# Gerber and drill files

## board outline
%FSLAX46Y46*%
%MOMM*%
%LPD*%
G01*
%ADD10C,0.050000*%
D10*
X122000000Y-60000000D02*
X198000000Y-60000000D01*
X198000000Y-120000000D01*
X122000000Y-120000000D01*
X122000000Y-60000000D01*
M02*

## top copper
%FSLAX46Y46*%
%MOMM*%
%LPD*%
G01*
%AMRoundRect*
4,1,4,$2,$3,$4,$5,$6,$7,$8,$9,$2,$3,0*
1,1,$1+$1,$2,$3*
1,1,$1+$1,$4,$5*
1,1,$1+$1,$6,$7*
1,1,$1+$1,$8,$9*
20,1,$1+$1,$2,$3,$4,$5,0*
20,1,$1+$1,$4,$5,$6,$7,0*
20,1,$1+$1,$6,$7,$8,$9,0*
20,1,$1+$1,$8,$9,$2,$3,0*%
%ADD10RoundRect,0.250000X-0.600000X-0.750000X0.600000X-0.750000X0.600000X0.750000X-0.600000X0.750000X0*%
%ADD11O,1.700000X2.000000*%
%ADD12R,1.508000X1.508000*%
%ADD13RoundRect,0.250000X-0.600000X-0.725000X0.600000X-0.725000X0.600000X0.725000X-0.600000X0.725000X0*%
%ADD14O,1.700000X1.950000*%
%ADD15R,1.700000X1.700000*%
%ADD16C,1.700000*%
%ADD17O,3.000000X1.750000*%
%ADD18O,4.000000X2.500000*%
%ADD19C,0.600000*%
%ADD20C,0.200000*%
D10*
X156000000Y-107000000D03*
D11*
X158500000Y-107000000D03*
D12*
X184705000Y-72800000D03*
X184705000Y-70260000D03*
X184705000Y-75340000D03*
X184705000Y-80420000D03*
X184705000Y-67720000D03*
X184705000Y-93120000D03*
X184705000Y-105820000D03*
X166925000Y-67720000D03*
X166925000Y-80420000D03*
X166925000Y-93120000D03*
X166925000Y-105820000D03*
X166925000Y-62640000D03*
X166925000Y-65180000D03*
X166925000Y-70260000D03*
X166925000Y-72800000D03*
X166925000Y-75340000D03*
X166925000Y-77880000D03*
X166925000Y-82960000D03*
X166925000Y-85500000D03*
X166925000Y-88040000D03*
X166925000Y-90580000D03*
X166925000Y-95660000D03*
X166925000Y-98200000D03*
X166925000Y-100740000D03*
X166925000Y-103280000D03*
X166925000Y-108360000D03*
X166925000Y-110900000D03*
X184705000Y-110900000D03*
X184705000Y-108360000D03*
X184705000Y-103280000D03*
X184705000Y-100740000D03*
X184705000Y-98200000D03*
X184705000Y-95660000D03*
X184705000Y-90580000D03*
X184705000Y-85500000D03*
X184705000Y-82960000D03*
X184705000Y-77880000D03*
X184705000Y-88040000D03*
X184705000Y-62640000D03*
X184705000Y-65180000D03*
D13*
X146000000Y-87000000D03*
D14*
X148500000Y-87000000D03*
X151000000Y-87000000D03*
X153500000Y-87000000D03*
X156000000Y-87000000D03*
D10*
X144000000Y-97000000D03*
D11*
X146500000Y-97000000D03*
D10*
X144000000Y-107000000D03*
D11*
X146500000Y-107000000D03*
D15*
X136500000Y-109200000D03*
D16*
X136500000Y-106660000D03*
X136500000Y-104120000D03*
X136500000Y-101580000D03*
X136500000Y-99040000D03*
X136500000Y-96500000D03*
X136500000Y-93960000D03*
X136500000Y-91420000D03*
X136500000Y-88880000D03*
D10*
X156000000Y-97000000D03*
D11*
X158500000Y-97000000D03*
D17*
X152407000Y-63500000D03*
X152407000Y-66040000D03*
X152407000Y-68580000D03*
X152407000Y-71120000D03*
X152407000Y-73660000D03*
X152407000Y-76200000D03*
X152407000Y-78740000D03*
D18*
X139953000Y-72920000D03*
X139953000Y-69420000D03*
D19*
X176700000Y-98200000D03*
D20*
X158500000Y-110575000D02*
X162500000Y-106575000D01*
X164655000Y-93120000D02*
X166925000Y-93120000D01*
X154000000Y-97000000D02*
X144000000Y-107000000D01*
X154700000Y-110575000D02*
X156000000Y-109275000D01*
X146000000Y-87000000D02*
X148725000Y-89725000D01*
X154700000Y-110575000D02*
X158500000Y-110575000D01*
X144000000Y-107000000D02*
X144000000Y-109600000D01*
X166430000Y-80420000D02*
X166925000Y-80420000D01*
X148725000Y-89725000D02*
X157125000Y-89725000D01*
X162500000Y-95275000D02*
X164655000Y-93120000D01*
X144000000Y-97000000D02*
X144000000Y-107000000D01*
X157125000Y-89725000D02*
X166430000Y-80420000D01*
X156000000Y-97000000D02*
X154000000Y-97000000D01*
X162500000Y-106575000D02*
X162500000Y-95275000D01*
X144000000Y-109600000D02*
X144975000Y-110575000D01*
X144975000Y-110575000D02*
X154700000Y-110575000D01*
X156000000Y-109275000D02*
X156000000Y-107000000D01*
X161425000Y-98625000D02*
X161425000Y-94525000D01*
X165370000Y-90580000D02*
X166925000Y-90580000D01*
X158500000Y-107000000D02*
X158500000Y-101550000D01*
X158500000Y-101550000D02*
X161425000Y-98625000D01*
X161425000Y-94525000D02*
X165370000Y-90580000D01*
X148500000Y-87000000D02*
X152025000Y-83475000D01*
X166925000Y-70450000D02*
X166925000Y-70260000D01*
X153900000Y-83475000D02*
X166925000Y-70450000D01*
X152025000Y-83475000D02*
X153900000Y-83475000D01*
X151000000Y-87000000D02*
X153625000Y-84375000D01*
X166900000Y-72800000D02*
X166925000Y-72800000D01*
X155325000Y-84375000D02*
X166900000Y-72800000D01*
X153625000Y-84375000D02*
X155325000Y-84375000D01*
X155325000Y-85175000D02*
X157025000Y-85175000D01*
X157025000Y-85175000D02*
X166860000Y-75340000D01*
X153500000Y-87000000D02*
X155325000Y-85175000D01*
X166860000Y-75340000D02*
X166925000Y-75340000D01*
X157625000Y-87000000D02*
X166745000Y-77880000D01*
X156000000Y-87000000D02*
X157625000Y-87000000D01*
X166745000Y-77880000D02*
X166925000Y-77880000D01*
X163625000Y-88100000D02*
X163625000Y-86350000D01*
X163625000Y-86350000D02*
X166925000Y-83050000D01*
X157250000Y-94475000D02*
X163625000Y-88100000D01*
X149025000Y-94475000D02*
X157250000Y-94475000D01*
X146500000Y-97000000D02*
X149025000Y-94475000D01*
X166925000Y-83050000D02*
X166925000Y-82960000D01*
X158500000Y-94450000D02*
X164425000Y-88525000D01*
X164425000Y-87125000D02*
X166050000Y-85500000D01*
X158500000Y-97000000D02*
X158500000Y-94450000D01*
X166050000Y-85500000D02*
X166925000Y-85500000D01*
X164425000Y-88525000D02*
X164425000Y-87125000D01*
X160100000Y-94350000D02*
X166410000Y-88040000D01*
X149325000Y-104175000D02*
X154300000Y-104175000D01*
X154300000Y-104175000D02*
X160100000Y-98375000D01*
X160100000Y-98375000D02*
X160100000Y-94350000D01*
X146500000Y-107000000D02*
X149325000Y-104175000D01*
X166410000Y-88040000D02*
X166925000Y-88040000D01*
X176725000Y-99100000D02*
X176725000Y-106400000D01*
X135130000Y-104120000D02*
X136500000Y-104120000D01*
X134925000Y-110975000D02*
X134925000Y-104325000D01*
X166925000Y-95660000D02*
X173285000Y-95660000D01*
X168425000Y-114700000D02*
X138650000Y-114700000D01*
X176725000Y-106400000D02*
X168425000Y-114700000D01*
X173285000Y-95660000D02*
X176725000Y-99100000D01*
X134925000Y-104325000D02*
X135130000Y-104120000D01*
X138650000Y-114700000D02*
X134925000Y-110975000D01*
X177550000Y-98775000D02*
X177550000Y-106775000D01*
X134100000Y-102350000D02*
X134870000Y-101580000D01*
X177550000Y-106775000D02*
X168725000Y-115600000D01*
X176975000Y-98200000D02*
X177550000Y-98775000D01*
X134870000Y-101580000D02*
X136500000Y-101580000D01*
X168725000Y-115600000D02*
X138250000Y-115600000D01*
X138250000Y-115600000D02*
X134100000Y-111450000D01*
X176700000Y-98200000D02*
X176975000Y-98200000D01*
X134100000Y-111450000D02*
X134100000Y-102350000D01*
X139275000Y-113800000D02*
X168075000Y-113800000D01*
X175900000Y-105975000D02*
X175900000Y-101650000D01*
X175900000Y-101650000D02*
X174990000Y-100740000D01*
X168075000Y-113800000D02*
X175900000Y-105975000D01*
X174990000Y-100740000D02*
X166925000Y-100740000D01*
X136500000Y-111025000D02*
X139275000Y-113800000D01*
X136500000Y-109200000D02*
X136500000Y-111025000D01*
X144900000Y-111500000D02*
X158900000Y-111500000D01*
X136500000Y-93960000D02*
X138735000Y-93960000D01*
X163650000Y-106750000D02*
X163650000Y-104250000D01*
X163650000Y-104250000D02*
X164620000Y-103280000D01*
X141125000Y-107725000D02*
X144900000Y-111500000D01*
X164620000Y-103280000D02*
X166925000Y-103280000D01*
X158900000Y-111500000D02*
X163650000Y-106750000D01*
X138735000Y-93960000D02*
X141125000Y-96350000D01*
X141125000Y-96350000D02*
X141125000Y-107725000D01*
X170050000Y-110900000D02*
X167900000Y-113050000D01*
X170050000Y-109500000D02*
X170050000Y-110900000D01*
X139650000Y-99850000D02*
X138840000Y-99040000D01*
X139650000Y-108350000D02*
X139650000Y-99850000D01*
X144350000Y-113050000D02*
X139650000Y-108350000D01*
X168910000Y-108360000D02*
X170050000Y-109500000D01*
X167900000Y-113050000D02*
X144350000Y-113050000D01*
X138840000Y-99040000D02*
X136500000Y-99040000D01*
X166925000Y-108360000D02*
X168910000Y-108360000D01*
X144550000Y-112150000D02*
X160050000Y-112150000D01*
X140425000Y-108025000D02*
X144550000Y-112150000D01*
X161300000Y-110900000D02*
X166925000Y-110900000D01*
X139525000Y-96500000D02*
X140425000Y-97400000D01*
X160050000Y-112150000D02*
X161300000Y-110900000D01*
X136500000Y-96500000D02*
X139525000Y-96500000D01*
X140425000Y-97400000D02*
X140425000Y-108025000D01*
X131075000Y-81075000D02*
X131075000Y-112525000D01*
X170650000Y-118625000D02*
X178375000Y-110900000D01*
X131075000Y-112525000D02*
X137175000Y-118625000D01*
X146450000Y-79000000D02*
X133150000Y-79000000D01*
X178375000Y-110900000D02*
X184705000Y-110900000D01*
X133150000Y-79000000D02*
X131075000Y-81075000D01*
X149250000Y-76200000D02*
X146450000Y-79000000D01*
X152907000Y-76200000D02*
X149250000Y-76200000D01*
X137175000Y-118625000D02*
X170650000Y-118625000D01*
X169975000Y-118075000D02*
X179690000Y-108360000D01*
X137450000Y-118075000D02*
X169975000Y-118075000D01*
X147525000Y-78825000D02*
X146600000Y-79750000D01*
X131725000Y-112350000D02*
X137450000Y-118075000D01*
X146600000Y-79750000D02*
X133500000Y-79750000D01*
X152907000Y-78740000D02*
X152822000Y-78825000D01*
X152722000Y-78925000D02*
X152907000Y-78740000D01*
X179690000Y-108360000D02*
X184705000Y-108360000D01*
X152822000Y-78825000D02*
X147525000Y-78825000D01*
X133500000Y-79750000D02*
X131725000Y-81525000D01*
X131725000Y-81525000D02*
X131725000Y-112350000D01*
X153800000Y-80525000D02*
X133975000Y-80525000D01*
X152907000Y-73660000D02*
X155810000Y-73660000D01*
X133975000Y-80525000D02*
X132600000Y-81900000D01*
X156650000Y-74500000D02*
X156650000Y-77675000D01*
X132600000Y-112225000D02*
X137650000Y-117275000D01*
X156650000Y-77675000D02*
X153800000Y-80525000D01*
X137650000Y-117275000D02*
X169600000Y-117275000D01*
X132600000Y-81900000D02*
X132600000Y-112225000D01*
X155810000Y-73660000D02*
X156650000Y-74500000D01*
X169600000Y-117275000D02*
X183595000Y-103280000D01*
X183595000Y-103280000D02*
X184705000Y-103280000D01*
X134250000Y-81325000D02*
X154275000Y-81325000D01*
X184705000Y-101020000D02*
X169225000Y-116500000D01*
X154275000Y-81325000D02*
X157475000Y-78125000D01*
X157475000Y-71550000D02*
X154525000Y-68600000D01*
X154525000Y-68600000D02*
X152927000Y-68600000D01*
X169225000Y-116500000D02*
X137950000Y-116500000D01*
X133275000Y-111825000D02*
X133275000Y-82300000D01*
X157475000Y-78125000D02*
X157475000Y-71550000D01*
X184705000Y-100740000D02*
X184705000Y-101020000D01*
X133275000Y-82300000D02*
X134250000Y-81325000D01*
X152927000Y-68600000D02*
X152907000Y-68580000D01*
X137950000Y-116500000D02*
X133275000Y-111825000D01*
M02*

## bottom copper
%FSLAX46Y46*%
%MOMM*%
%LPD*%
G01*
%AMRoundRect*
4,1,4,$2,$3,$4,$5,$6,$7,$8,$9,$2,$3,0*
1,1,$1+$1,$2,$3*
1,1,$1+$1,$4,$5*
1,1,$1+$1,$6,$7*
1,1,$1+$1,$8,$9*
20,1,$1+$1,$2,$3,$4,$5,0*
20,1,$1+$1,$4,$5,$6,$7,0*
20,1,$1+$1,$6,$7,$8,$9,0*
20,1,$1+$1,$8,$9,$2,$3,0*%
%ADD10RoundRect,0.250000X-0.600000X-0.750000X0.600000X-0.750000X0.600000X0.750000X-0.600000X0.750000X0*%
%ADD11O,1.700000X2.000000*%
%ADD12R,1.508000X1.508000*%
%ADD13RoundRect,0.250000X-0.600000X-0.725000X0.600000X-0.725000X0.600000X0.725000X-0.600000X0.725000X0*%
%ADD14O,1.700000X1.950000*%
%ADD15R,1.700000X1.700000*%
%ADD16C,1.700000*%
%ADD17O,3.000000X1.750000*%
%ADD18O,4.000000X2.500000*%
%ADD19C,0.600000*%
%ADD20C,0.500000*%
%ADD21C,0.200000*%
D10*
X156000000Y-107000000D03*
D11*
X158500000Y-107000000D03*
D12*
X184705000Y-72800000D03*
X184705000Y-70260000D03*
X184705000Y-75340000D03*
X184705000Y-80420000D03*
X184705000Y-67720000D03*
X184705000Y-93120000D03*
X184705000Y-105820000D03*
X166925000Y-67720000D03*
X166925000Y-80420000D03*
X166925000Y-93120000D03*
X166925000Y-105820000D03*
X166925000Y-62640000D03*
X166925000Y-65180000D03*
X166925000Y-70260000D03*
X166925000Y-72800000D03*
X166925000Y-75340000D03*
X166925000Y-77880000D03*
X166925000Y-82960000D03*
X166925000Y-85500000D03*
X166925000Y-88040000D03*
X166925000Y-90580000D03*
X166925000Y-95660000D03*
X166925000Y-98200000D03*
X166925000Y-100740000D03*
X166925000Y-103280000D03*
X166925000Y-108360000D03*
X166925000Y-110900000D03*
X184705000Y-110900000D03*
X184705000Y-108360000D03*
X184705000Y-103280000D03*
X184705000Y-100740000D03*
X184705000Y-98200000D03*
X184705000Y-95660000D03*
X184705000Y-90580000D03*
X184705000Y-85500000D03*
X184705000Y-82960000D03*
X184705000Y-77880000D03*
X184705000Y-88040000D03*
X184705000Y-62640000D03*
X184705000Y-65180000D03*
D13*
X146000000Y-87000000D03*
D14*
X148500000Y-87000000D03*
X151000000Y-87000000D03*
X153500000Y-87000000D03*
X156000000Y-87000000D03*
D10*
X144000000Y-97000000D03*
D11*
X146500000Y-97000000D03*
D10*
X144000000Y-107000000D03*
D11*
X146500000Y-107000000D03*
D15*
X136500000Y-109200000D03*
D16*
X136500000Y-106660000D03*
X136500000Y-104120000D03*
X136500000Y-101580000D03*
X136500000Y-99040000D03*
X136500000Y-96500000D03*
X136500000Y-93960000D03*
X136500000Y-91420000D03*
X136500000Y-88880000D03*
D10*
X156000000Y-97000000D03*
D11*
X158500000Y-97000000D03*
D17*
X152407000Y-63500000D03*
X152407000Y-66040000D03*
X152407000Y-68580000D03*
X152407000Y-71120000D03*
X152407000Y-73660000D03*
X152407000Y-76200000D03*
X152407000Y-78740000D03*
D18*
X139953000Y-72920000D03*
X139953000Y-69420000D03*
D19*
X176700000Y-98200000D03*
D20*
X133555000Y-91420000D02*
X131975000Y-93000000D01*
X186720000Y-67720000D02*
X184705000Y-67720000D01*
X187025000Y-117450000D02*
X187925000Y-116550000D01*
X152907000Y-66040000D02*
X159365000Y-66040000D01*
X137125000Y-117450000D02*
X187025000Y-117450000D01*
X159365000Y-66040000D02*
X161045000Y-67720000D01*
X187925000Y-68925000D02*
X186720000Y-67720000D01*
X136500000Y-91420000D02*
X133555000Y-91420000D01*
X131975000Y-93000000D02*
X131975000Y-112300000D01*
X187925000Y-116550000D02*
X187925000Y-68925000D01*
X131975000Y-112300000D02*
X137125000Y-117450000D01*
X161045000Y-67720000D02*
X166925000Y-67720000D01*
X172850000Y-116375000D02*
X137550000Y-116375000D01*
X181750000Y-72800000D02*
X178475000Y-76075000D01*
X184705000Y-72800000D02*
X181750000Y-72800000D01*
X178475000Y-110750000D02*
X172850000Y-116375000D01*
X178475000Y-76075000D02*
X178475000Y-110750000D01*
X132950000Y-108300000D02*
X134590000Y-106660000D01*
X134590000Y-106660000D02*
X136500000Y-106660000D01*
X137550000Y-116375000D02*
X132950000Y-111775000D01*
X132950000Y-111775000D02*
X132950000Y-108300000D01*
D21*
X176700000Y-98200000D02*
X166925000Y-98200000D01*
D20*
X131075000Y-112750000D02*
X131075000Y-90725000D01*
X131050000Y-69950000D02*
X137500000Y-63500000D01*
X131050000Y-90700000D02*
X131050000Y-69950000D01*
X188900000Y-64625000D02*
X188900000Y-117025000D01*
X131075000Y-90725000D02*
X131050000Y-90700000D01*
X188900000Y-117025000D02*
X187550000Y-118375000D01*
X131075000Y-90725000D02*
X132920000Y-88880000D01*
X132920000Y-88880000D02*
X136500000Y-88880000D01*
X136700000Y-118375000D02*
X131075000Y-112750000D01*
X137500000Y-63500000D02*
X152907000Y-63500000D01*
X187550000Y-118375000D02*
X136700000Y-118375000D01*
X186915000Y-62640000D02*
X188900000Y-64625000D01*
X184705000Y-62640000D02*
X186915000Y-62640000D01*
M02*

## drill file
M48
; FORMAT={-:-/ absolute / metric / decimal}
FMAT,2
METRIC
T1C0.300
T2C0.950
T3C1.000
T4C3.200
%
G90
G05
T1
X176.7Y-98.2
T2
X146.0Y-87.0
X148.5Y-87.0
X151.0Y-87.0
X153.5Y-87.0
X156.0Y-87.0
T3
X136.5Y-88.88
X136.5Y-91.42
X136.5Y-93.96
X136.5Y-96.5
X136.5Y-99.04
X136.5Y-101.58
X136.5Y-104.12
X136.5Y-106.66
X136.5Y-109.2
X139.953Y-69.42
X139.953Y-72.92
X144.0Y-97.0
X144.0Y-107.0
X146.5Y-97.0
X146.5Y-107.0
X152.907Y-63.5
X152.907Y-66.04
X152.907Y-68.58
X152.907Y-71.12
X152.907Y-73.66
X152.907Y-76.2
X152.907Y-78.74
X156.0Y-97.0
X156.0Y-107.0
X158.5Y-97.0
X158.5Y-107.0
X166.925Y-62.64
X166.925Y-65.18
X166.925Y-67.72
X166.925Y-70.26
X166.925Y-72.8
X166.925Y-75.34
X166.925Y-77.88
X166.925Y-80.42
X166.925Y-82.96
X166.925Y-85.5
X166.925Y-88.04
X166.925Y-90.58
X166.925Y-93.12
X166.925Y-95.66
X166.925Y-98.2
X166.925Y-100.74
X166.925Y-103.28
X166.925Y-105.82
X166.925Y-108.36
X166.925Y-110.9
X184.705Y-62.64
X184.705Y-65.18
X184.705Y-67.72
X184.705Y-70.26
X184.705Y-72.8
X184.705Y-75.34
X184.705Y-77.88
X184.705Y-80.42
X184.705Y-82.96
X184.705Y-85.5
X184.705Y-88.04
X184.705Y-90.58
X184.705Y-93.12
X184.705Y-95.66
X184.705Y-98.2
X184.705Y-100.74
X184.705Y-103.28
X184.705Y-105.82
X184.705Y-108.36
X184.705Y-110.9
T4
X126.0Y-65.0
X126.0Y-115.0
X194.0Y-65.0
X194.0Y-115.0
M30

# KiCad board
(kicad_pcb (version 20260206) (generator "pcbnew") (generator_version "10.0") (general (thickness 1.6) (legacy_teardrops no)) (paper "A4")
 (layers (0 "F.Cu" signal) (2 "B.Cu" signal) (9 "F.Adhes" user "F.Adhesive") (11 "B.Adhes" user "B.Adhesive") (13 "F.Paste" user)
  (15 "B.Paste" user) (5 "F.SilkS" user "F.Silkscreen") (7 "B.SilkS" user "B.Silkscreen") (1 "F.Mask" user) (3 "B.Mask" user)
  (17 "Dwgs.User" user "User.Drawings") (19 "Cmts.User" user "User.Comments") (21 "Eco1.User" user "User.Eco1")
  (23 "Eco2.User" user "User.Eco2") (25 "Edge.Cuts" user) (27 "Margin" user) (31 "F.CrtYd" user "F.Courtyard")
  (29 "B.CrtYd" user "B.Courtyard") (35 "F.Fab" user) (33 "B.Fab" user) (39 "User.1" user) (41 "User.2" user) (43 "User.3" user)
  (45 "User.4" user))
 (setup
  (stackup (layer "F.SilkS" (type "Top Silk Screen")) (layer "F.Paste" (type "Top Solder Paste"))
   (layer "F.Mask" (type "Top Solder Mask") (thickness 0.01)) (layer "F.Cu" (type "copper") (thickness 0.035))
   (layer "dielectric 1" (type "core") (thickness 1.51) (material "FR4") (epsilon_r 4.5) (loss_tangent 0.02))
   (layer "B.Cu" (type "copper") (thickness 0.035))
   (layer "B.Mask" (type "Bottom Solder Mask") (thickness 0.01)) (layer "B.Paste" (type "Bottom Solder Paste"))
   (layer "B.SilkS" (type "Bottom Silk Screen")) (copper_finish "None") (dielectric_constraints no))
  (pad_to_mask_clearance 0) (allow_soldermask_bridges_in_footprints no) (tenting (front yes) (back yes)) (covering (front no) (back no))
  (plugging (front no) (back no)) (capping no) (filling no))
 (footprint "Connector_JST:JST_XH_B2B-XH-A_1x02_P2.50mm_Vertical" (layer "F.Cu") (at 156 107)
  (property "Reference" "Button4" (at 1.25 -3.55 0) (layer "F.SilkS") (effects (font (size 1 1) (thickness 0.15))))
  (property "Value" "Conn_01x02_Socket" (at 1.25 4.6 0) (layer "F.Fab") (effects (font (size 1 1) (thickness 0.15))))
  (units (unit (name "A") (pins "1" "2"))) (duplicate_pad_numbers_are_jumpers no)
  (pad "1" thru_hole roundrect (at 0 0) (size 1.7 2) (drill 1) (layers "*.Cu" "*.Mask") (remove_unused_layers no)
   (roundrect_rratio 0.147059) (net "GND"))
  (pad "2" thru_hole oval (at 2.5 0) (size 1.7 2) (drill 1) (layers "*.Cu" "*.Mask") (remove_unused_layers no) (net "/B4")))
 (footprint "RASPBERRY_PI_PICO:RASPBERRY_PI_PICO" (layer "F.Cu") (at 175.815 85.5)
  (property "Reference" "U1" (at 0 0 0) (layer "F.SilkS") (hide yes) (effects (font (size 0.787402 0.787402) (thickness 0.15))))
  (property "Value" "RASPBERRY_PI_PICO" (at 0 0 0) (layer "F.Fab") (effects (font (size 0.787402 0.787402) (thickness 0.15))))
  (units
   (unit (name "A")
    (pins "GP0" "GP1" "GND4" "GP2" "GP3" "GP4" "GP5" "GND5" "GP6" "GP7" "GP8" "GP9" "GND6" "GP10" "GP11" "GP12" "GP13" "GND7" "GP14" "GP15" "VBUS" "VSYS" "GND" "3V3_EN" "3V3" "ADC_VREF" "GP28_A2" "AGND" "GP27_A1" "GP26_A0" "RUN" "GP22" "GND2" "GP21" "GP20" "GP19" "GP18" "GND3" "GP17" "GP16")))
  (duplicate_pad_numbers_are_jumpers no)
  (pad "3V3" thru_hole rect (at 8.89 -12.7) (size 1.508 1.508) (drill 1) (layers "*.Cu" "*.Mask") (remove_unused_layers no) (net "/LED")
   (solder_mask_margin 0.102))
  (pad "3V3_EN" thru_hole rect (at 8.89 -15.24) (size 1.508 1.508) (drill 1) (layers "*.Cu" "*.Mask") (remove_unused_layers no)
   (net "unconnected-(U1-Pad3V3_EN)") (solder_mask_margin 0.102))
  (pad "ADC_VREF" thru_hole rect (at 8.89 -10.16) (size 1.508 1.508) (drill 1) (layers "*.Cu" "*.Mask") (remove_unused_layers no)
   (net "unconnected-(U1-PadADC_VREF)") (solder_mask_margin 0.102))
  (pad "AGND" thru_hole rect (at 8.89 -5.08) (size 1.508 1.508) (drill 1) (layers "*.Cu" "*.Mask") (remove_unused_layers no)
   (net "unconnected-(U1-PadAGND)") (solder_mask_margin 0.102))
  (pad "GND" thru_hole rect (at 8.89 -17.78) (size 1.508 1.508) (drill 1) (layers "*.Cu" "*.Mask") (remove_unused_layers no) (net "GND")
   (solder_mask_margin 0.102))
  (pad "GND2" thru_hole rect (at 8.89 7.62) (size 1.508 1.508) (drill 1) (layers "*.Cu" "*.Mask") (remove_unused_layers no)
   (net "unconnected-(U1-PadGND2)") (solder_mask_margin 0.102))
  (pad "GND3" thru_hole rect (at 8.89 20.32) (size 1.508 1.508) (drill 1) (layers "*.Cu" "*.Mask") (remove_unused_layers no)
   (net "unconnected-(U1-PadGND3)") (solder_mask_margin 0.102))
  (pad "GND4" thru_hole rect (at -8.89 -17.78) (size 1.508 1.508) (drill 1) (layers "*.Cu" "*.Mask") (remove_unused_layers no) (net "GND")
   (solder_mask_margin 0.102))
  (pad "GND5" thru_hole rect (at -8.89 -5.08) (size 1.508 1.508) (drill 1) (layers "*.Cu" "*.Mask") (remove_unused_layers no) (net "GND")
   (solder_mask_margin 0.102))
  (pad "GND6" thru_hole rect (at -8.89 7.62) (size 1.508 1.508) (drill 1) (layers "*.Cu" "*.Mask") (remove_unused_layers no) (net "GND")
   (solder_mask_margin 0.102))
  (pad "GND7" thru_hole rect (at -8.89 20.32) (size 1.508 1.508) (drill 1) (layers "*.Cu" "*.Mask") (remove_unused_layers no)
   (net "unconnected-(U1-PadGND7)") (solder_mask_margin 0.102))
  (pad "GP0" thru_hole rect (at -8.89 -22.86) (size 1.508 1.508) (drill 1) (layers "*.Cu" "*.Mask") (remove_unused_layers no)
   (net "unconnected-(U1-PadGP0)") (solder_mask_margin 0.102))
  (pad "GP1" thru_hole rect (at -8.89 -20.32) (size 1.508 1.508) (drill 1) (layers "*.Cu" "*.Mask") (remove_unused_layers no)
   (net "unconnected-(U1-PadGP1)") (solder_mask_margin 0.102))
  (pad "GP2" thru_hole rect (at -8.89 -15.24) (size 1.508 1.508) (drill 1) (layers "*.Cu" "*.Mask") (remove_unused_layers no) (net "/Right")
   (solder_mask_margin 0.102))
  (pad "GP3" thru_hole rect (at -8.89 -12.7) (size 1.508 1.508) (drill 1) (layers "*.Cu" "*.Mask") (remove_unused_layers no) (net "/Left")
   (solder_mask_margin 0.102))
  (pad "GP4" thru_hole rect (at -8.89 -10.16) (size 1.508 1.508) (drill 1) (layers "*.Cu" "*.Mask") (remove_unused_layers no) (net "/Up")
   (solder_mask_margin 0.102))
  (pad "GP5" thru_hole rect (at -8.89 -7.62) (size 1.508 1.508) (drill 1) (layers "*.Cu" "*.Mask") (remove_unused_layers no) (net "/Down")
   (solder_mask_margin 0.102))
  (pad "GP6" thru_hole rect (at -8.89 -2.54) (size 1.508 1.508) (drill 1) (layers "*.Cu" "*.Mask") (remove_unused_layers no) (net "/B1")
   (solder_mask_margin 0.102))
  (pad "GP7" thru_hole rect (at -8.89 0) (size 1.508 1.508) (drill 1) (layers "*.Cu" "*.Mask") (remove_unused_layers no) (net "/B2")
   (solder_mask_margin 0.102))
  (pad "GP8" thru_hole rect (at -8.89 2.54) (size 1.508 1.508) (drill 1) (layers "*.Cu" "*.Mask") (remove_unused_layers no) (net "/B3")
   (solder_mask_margin 0.102))
  (pad "GP9" thru_hole rect (at -8.89 5.08) (size 1.508 1.508) (drill 1) (layers "*.Cu" "*.Mask") (remove_unused_layers no) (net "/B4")
   (solder_mask_margin 0.102))
  (pad "GP10" thru_hole rect (at -8.89 10.16) (size 1.508 1.508) (drill 1) (layers "*.Cu" "*.Mask") (remove_unused_layers no) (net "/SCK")
   (solder_mask_margin 0.102))
  (pad "GP11" thru_hole rect (at -8.89 12.7) (size 1.508 1.508) (drill 1) (layers "*.Cu" "*.Mask") (remove_unused_layers no) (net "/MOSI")
   (solder_mask_margin 0.102))
  (pad "GP12" thru_hole rect (at -8.89 15.24) (size 1.508 1.508) (drill 1) (layers "*.Cu" "*.Mask") (remove_unused_layers no) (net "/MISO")
   (solder_mask_margin 0.102))
  (pad "GP13" thru_hole rect (at -8.89 17.78) (size 1.508 1.508) (drill 1) (layers "*.Cu" "*.Mask") (remove_unused_layers no) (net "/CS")
   (solder_mask_margin 0.102))
  (pad "GP14" thru_hole rect (at -8.89 22.86) (size 1.508 1.508) (drill 1) (layers "*.Cu" "*.Mask") (remove_unused_layers no)
   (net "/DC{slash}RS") (solder_mask_margin 0.102))
  (pad "GP15" thru_hole rect (at -8.89 25.4) (size 1.508 1.508) (drill 1) (layers "*.Cu" "*.Mask") (remove_unused_layers no) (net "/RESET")
   (solder_mask_margin 0.102))
  (pad "GP16" thru_hole rect (at 8.89 25.4) (size 1.508 1.508) (drill 1) (layers "*.Cu" "*.Mask") (remove_unused_layers no) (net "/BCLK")
   (solder_mask_margin 0.102))
  (pad "GP17" thru_hole rect (at 8.89 22.86) (size 1.508 1.508) (drill 1) (layers "*.Cu" "*.Mask") (remove_unused_layers no) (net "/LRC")
   (solder_mask_margin 0.102))
  (pad "GP18" thru_hole rect (at 8.89 17.78) (size 1.508 1.508) (drill 1) (layers "*.Cu" "*.Mask") (remove_unused_layers no) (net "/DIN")
   (solder_mask_margin 0.102))
  (pad "GP19" thru_hole rect (at 8.89 15.24) (size 1.508 1.508) (drill 1) (layers "*.Cu" "*.Mask") (remove_unused_layers no)
   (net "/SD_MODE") (solder_mask_margin 0.102))
  (pad "GP20" thru_hole rect (at 8.89 12.7) (size 1.508 1.508) (drill 1) (layers "*.Cu" "*.Mask") (remove_unused_layers no)
   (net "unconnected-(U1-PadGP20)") (solder_mask_margin 0.102))
  (pad "GP21" thru_hole rect (at 8.89 10.16) (size 1.508 1.508) (drill 1) (layers "*.Cu" "*.Mask") (remove_unused_layers no)
   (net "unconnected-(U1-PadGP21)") (solder_mask_margin 0.102))
  (pad "GP22" thru_hole rect (at 8.89 5.08) (size 1.508 1.508) (drill 1) (layers "*.Cu" "*.Mask") (remove_unused_layers no)
   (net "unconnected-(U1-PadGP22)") (solder_mask_margin 0.102))
  (pad "GP26_A0" thru_hole rect (at 8.89 0) (size 1.508 1.508) (drill 1) (layers "*.Cu" "*.Mask") (remove_unused_layers no)
   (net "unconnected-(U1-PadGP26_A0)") (solder_mask_margin 0.102))
  (pad "GP27_A1" thru_hole rect (at 8.89 -2.54) (size 1.508 1.508) (drill 1) (layers "*.Cu" "*.Mask") (remove_unused_layers no)
   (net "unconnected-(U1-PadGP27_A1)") (solder_mask_margin 0.102))
  (pad "GP28_A2" thru_hole rect (at 8.89 -7.62) (size 1.508 1.508) (drill 1) (layers "*.Cu" "*.Mask") (remove_unused_layers no)
   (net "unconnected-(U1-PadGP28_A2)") (solder_mask_margin 0.102))
  (pad "RUN" thru_hole rect (at 8.89 2.54) (size 1.508 1.508) (drill 1) (layers "*.Cu" "*.Mask") (remove_unused_layers no)
   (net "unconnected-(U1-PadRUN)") (solder_mask_margin 0.102))
  (pad "VBUS" thru_hole rect (at 8.89 -22.86) (size 1.508 1.508) (drill 1) (layers "*.Cu" "*.Mask") (remove_unused_layers no) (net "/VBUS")
   (solder_mask_margin 0.102))
  (pad "VSYS" thru_hole rect (at 8.89 -20.32) (size 1.508 1.508) (drill 1) (layers "*.Cu" "*.Mask") (remove_unused_layers no)
   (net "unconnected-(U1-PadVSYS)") (solder_mask_margin 0.102)))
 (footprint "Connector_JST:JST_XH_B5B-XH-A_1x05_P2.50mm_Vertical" (layer "F.Cu") (at 146 87)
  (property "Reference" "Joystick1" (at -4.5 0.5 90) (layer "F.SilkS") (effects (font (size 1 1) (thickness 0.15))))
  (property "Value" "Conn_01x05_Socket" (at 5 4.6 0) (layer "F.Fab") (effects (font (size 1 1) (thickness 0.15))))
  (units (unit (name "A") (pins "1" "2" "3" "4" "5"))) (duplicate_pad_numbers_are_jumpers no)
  (pad "1" thru_hole roundrect (at 0 0) (size 1.7 1.95) (drill 0.95) (layers "*.Cu" "*.Mask") (remove_unused_layers no)
   (roundrect_rratio 0.147059) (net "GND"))
  (pad "2" thru_hole oval (at 2.5 0) (size 1.7 1.95) (drill 0.95) (layers "*.Cu" "*.Mask") (remove_unused_layers no) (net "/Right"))
  (pad "3" thru_hole oval (at 5 0) (size 1.7 1.95) (drill 0.95) (layers "*.Cu" "*.Mask") (remove_unused_layers no) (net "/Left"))
  (pad "4" thru_hole oval (at 7.5 0) (size 1.7 1.95) (drill 0.95) (layers "*.Cu" "*.Mask") (remove_unused_layers no) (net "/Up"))
  (pad "5" thru_hole oval (at 10 0) (size 1.7 1.95) (drill 0.95) (layers "*.Cu" "*.Mask") (remove_unused_layers no) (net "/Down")))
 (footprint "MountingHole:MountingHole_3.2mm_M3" (layer "F.Cu") (at 126 115)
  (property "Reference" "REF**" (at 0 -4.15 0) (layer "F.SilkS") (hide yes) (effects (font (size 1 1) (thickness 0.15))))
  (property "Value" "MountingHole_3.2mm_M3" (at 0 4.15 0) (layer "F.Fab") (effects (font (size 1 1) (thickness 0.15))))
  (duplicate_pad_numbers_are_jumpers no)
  (pad "" np_thru_hole circle (at 0 0) (size 3.2 3.2) (drill 3.2) (layers "*.Cu" "*.Mask")))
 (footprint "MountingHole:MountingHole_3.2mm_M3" (layer "F.Cu") (at 194 65)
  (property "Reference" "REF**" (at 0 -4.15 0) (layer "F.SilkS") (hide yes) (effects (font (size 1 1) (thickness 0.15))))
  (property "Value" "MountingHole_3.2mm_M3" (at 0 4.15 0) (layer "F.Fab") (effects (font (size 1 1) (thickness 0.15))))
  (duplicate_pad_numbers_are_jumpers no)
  (pad "" np_thru_hole circle (at 0 0) (size 3.2 3.2) (drill 3.2) (layers "*.Cu" "*.Mask")))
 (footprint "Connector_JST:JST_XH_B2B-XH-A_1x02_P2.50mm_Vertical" (layer "F.Cu") (at 144 97)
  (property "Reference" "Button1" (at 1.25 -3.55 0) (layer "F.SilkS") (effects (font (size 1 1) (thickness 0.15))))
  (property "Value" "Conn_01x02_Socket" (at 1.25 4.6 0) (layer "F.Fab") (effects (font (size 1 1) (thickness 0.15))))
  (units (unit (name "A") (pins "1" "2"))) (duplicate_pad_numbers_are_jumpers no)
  (pad "1" thru_hole roundrect (at 0 0) (size 1.7 2) (drill 1) (layers "*.Cu" "*.Mask") (remove_unused_layers no)
   (roundrect_rratio 0.147059) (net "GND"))
  (pad "2" thru_hole oval (at 2.5 0) (size 1.7 2) (drill 1) (layers "*.Cu" "*.Mask") (remove_unused_layers no) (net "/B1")))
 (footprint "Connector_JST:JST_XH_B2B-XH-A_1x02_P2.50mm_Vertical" (layer "F.Cu") (at 144 107)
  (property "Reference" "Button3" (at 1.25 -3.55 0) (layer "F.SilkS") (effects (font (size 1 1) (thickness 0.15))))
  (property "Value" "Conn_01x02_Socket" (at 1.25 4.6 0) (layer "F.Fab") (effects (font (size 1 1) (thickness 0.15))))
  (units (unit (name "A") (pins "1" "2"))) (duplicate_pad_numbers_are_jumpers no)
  (pad "1" thru_hole roundrect (at 0 0) (size 1.7 2) (drill 1) (layers "*.Cu" "*.Mask") (remove_unused_layers no)
   (roundrect_rratio 0.147059) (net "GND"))
  (pad "2" thru_hole oval (at 2.5 0) (size 1.7 2) (drill 1) (layers "*.Cu" "*.Mask") (remove_unused_layers no) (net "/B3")))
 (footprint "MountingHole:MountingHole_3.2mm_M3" (layer "F.Cu") (at 194 115)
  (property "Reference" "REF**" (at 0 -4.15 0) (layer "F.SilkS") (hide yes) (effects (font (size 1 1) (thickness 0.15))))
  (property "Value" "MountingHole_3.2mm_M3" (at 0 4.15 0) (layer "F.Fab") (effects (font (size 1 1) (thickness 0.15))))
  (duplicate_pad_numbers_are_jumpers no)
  (pad "" np_thru_hole circle (at 0 0) (size 3.2 3.2) (drill 3.2) (layers "*.Cu" "*.Mask")))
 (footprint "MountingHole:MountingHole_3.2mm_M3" (layer "F.Cu") (at 126 65)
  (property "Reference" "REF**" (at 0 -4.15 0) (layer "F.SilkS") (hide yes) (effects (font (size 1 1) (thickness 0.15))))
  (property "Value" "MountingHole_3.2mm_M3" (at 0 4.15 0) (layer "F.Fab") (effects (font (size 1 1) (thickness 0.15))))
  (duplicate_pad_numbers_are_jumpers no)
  (pad "" np_thru_hole circle (at 0 0) (size 3.2 3.2) (drill 3.2) (layers "*.Cu" "*.Mask")))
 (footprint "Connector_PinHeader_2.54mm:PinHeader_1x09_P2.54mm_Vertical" (layer "F.Cu") (at 136.5 109.2 180)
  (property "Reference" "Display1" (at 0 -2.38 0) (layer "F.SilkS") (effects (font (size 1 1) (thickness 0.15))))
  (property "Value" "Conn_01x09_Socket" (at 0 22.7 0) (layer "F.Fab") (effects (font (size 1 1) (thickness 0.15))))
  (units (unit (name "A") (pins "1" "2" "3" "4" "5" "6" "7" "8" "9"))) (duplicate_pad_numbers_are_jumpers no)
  (pad "1" thru_hole rect (at 0 0 180) (size 1.7 1.7) (drill 1) (layers "*.Cu" "*.Mask") (remove_unused_layers no) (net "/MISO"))
  (pad "2" thru_hole circle (at 0 2.54 180) (size 1.7 1.7) (drill 1) (layers "*.Cu" "*.Mask") (remove_unused_layers no) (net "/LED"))
  (pad "3" thru_hole circle (at 0 5.08 180) (size 1.7 1.7) (drill 1) (layers "*.Cu" "*.Mask") (remove_unused_layers no) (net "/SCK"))
  (pad "4" thru_hole circle (at 0 7.62 180) (size 1.7 1.7) (drill 1) (layers "*.Cu" "*.Mask") (remove_unused_layers no) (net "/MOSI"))
  (pad "5" thru_hole circle (at 0 10.16 180) (size 1.7 1.7) (drill 1) (layers "*.Cu" "*.Mask") (remove_unused_layers no)
   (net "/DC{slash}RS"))
  (pad "6" thru_hole circle (at 0 12.7 180) (size 1.7 1.7) (drill 1) (layers "*.Cu" "*.Mask") (remove_unused_layers no) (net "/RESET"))
  (pad "7" thru_hole circle (at 0 15.24 180) (size 1.7 1.7) (drill 1) (layers "*.Cu" "*.Mask") (remove_unused_layers no) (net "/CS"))
  (pad "8" thru_hole circle (at 0 17.78 180) (size 1.7 1.7) (drill 1) (layers "*.Cu" "*.Mask") (remove_unused_layers no) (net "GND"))
  (pad "9" thru_hole circle (at 0 20.32 180) (size 1.7 1.7) (drill 1) (layers "*.Cu" "*.Mask") (remove_unused_layers no) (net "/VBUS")))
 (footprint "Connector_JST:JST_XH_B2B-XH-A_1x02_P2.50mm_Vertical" (layer "F.Cu") (at 156 97)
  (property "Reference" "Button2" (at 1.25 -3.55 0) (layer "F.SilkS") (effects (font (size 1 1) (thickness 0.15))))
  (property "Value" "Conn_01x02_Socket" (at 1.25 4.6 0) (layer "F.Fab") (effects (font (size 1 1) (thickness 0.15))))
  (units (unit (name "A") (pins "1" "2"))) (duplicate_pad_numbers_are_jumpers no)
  (pad "1" thru_hole roundrect (at 0 0) (size 1.7 2) (drill 1) (layers "*.Cu" "*.Mask") (remove_unused_layers no)
   (roundrect_rratio 0.147059) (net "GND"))
  (pad "2" thru_hole oval (at 2.5 0) (size 1.7 2) (drill 1) (layers "*.Cu" "*.Mask") (remove_unused_layers no) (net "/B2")))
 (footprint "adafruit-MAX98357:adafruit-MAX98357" (layer "F.Cu") (at 146 71 90)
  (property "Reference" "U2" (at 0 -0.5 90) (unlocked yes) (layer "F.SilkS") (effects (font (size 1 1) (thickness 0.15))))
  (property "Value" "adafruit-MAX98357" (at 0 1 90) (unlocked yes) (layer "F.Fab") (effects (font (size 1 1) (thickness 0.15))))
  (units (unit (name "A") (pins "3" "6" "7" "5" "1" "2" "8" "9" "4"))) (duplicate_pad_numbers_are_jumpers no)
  (pad "1" thru_hole oval (at 7.5 6.907) (size 3 1.75) (drill 1 (offset -0.5 0)) (layers "*.Cu" "*.Mask") (remove_unused_layers no)
   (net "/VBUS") (solder_mask_margin 0.0508))
  (pad "2" thru_hole oval (at 4.96 6.907) (size 3 1.75) (drill 1 (offset -0.5 0)) (layers "*.Cu" "*.Mask") (remove_unused_layers no)
   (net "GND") (solder_mask_margin 0.0508))
  (pad "3" thru_hole oval (at 2.42 6.907) (size 3 1.75) (drill 1 (offset -0.5 0)) (layers "*.Cu" "*.Mask") (remove_unused_layers no)
   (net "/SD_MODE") (solder_mask_margin 0.0508))
  (pad "4" thru_hole oval (at -0.12 6.907) (size 3 1.75) (drill 1 (offset -0.5 0)) (layers "*.Cu" "*.Mask") (remove_unused_layers no)
   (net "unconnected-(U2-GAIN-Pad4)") (solder_mask_margin 0.0508))
  (pad "5" thru_hole oval (at -2.66 6.907) (size 3 1.75) (drill 1 (offset -0.5 0)) (layers "*.Cu" "*.Mask") (remove_unused_layers no)
   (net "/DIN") (solder_mask_margin 0.0508))
  (pad "6" thru_hole oval (at -5.2 6.907) (size 3 1.75) (drill 1 (offset -0.5 0)) (layers "*.Cu" "*.Mask") (remove_unused_layers no)
   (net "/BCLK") (solder_mask_margin 0.0508))
  (pad "7" thru_hole oval (at -7.74 6.907) (size 3 1.75) (drill 1 (offset -0.5 0)) (layers "*.Cu" "*.Mask") (remove_unused_layers no)
   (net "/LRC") (solder_mask_margin 0.0508))
  (pad "8" thru_hole oval (at -1.92 -6.047 270) (size 2.5 4) (drill 1) (layers "*.Cu" "*.Mask") (remove_unused_layers no)
   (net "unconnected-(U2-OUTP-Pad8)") (solder_mask_margin 0.0508))
  (pad "9" thru_hole oval (at 1.58 -6.047 270) (size 2.5 4) (drill 1) (layers "*.Cu" "*.Mask") (remove_unused_layers no)
   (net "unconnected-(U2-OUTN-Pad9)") (solder_mask_margin 0.0508)))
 (gr_rect (start 122 60) (end 198 120) (stroke (width 0.05) (type default)) (fill no) (layer "Edge.Cuts"))
 (segment (start 158.5 110.575) (end 162.5 106.575) (width 0.2) (layer "F.Cu") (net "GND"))
 (segment (start 164.655 93.12) (end 166.925 93.12) (width 0.2) (layer "F.Cu") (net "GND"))
 (segment (start 154 97) (end 144 107) (width 0.2) (layer "F.Cu") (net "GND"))
 (segment (start 154.7 110.575) (end 156 109.275) (width 0.2) (layer "F.Cu") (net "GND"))
 (segment (start 146 87) (end 148.725 89.725) (width 0.2) (layer "F.Cu") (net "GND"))
 (segment (start 154.7 110.575) (end 158.5 110.575) (width 0.2) (layer "F.Cu") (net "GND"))
 (segment (start 144 107) (end 144 109.6) (width 0.2) (layer "F.Cu") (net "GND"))
 (segment (start 166.43 80.42) (end 166.925 80.42) (width 0.2) (layer "F.Cu") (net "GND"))
 (segment (start 148.725 89.725) (end 157.125 89.725) (width 0.2) (layer "F.Cu") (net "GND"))
 (segment (start 162.5 95.275) (end 164.655 93.12) (width 0.2) (layer "F.Cu") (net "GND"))
 (segment (start 144 97) (end 144 107) (width 0.2) (layer "F.Cu") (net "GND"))
 (segment (start 157.125 89.725) (end 166.43 80.42) (width 0.2) (layer "F.Cu") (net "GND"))
 (segment (start 156 97) (end 154 97) (width 0.2) (layer "F.Cu") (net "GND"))
 (segment (start 162.5 106.575) (end 162.5 95.275) (width 0.2) (layer "F.Cu") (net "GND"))
 (segment (start 144 109.6) (end 144.975 110.575) (width 0.2) (layer "F.Cu") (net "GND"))
 (segment (start 144.975 110.575) (end 154.7 110.575) (width 0.2) (layer "F.Cu") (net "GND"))
 (segment (start 156 109.275) (end 156 107) (width 0.2) (layer "F.Cu") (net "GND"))
 (segment (start 133.555 91.42) (end 131.975 93) (width 0.5) (layer "B.Cu") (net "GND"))
 (segment (start 186.72 67.72) (end 184.705 67.72) (width 0.5) (layer "B.Cu") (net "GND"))
 (segment (start 187.025 117.45) (end 187.925 116.55) (width 0.5) (layer "B.Cu") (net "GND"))
 (segment (start 152.907 66.04) (end 159.365 66.04) (width 0.5) (layer "B.Cu") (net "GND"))
 (segment (start 137.125 117.45) (end 187.025 117.45) (width 0.5) (layer "B.Cu") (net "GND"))
 (segment (start 159.365 66.04) (end 161.045 67.72) (width 0.5) (layer "B.Cu") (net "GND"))
 (segment (start 187.925 68.925) (end 186.72 67.72) (width 0.5) (layer "B.Cu") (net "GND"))
 (segment (start 136.5 91.42) (end 133.555 91.42) (width 0.5) (layer "B.Cu") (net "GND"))
 (segment (start 131.975 93) (end 131.975 112.3) (width 0.5) (layer "B.Cu") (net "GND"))
 (segment (start 187.925 116.55) (end 187.925 68.925) (width 0.5) (layer "B.Cu") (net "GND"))
 (segment (start 131.975 112.3) (end 137.125 117.45) (width 0.5) (layer "B.Cu") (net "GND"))
 (segment (start 161.045 67.72) (end 166.925 67.72) (width 0.5) (layer "B.Cu") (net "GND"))
 (segment (start 161.425 98.625) (end 161.425 94.525) (width 0.2) (layer "F.Cu") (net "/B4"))
 (segment (start 165.37 90.58) (end 166.925 90.58) (width 0.2) (layer "F.Cu") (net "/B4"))
 (segment (start 158.5 107) (end 158.5 101.55) (width 0.2) (layer "F.Cu") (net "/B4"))
 (segment (start 158.5 101.55) (end 161.425 98.625) (width 0.2) (layer "F.Cu") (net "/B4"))
 (segment (start 161.425 94.525) (end 165.37 90.58) (width 0.2) (layer "F.Cu") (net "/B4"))
 (segment (start 172.85 116.375) (end 137.55 116.375) (width 0.5) (layer "B.Cu") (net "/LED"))
 (segment (start 181.75 72.8) (end 178.475 76.075) (width 0.5) (layer "B.Cu") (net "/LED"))
 (segment (start 184.705 72.8) (end 181.75 72.8) (width 0.5) (layer "B.Cu") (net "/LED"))
 (segment (start 178.475 110.75) (end 172.85 116.375) (width 0.5) (layer "B.Cu") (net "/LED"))
 (segment (start 178.475 76.075) (end 178.475 110.75) (width 0.5) (layer "B.Cu") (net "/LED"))
 (segment (start 132.95 108.3) (end 134.59 106.66) (width 0.5) (layer "B.Cu") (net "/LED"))
 (segment (start 134.59 106.66) (end 136.5 106.66) (width 0.5) (layer "B.Cu") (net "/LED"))
 (segment (start 137.55 116.375) (end 132.95 111.775) (width 0.5) (layer "B.Cu") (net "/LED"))
 (segment (start 132.95 111.775) (end 132.95 108.3) (width 0.5) (layer "B.Cu") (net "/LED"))
 (segment (start 148.5 87) (end 152.025 83.475) (width 0.2) (layer "F.Cu") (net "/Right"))
 (segment (start 166.925 70.45) (end 166.925 70.26) (width 0.2) (layer "F.Cu") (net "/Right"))
 (segment (start 153.9 83.475) (end 166.925 70.45) (width 0.2) (layer "F.Cu") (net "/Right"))
 (segment (start 152.025 83.475) (end 153.9 83.475) (width 0.2) (layer "F.Cu") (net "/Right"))
 (segment (start 151 87) (end 153.625 84.375) (width 0.2) (layer "F.Cu") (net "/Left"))
 (segment (start 166.9 72.8) (end 166.925 72.8) (width 0.2) (layer "F.Cu") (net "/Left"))
 (segment (start 155.325 84.375) (end 166.9 72.8) (width 0.2) (layer "F.Cu") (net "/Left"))
 (segment (start 153.625 84.375) (end 155.325 84.375) (width 0.2) (layer "F.Cu") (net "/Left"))
 (segment (start 155.325 85.175) (end 157.025 85.175) (width 0.2) (layer "F.Cu") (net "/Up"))
 (segment (start 157.025 85.175) (end 166.86 75.34) (width 0.2) (layer "F.Cu") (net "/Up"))
 (segment (start 153.5 87) (end 155.325 85.175) (width 0.2) (layer "F.Cu") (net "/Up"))
 (segment (start 166.86 75.34) (end 166.925 75.34) (width 0.2) (layer "F.Cu") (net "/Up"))
 (segment (start 157.625 87) (end 166.745 77.88) (width 0.2) (layer "F.Cu") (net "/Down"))
 (segment (start 156 87) (end 157.625 87) (width 0.2) (layer "F.Cu") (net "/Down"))
 (segment (start 166.745 77.88) (end 166.925 77.88) (width 0.2) (layer "F.Cu") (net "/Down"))
 (segment (start 163.625 88.1) (end 163.625 86.35) (width 0.2) (layer "F.Cu") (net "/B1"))
 (segment (start 163.625 86.35) (end 166.925 83.05) (width 0.2) (layer "F.Cu") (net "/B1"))
 (segment (start 157.25 94.475) (end 163.625 88.1) (width 0.2) (layer "F.Cu") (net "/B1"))
 (segment (start 149.025 94.475) (end 157.25 94.475) (width 0.2) (layer "F.Cu") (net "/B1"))
 (segment (start 146.5 97) (end 149.025 94.475) (width 0.2) (layer "F.Cu") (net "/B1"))
 (segment (start 166.925 83.05) (end 166.925 82.96) (width 0.2) (layer "F.Cu") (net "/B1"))
 (segment (start 158.5 94.45) (end 164.425 88.525) (width 0.2) (layer "F.Cu") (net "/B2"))
 (segment (start 164.425 87.125) (end 166.05 85.5) (width 0.2) (layer "F.Cu") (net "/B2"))
 (segment (start 158.5 97) (end 158.5 94.45) (width 0.2) (layer "F.Cu") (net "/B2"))
 (segment (start 166.05 85.5) (end 166.925 85.5) (width 0.2) (layer "F.Cu") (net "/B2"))
 (segment (start 164.425 88.525) (end 164.425 87.125) (width 0.2) (layer "F.Cu") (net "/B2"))
 (segment (start 160.1 94.35) (end 166.41 88.04) (width 0.2) (layer "F.Cu") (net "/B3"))
 (segment (start 149.325 104.175) (end 154.3 104.175) (width 0.2) (layer "F.Cu") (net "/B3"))
 (segment (start 154.3 104.175) (end 160.1 98.375) (width 0.2) (layer "F.Cu") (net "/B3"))
 (segment (start 160.1 98.375) (end 160.1 94.35) (width 0.2) (layer "F.Cu") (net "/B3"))
 (segment (start 146.5 107) (end 149.325 104.175) (width 0.2) (layer "F.Cu") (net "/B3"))
 (segment (start 166.41 88.04) (end 166.925 88.04) (width 0.2) (layer "F.Cu") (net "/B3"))
 (segment (start 176.725 99.1) (end 176.725 106.4) (width 0.2) (layer "F.Cu") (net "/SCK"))
 (segment (start 135.13 104.12) (end 136.5 104.12) (width 0.2) (layer "F.Cu") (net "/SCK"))
 (segment (start 134.925 110.975) (end 134.925 104.325) (width 0.2) (layer "F.Cu") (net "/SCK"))
 (segment (start 166.925 95.66) (end 173.285 95.66) (width 0.2) (layer "F.Cu") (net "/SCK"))
 (segment (start 168.425 114.7) (end 138.65 114.7) (width 0.2) (layer "F.Cu") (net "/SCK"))
 (segment (start 176.725 106.4) (end 168.425 114.7) (width 0.2) (layer "F.Cu") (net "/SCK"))
 (segment (start 173.285 95.66) (end 176.725 99.1) (width 0.2) (layer "F.Cu") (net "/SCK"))
 (segment (start 134.925 104.325) (end 135.13 104.12) (width 0.2) (layer "F.Cu") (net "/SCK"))
 (segment (start 138.65 114.7) (end 134.925 110.975) (width 0.2) (layer "F.Cu") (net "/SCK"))
 (segment (start 177.55 98.775) (end 177.55 106.775) (width 0.2) (layer "F.Cu") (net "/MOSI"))
 (segment (start 134.1 102.35) (end 134.87 101.58) (width 0.2) (layer "F.Cu") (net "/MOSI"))
 (segment (start 177.55 106.775) (end 168.725 115.6) (width 0.2) (layer "F.Cu") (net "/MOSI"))
 (segment (start 176.975 98.2) (end 177.55 98.775) (width 0.2) (layer "F.Cu") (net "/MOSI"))
 (segment (start 134.87 101.58) (end 136.5 101.58) (width 0.2) (layer "F.Cu") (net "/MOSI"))
 (segment (start 168.725 115.6) (end 138.25 115.6) (width 0.2) (layer "F.Cu") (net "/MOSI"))
 (segment (start 138.25 115.6) (end 134.1 111.45) (width 0.2) (layer "F.Cu") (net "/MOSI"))
 (segment (start 176.7 98.2) (end 176.975 98.2) (width 0.2) (layer "F.Cu") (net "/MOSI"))
 (segment (start 134.1 111.45) (end 134.1 102.35) (width 0.2) (layer "F.Cu") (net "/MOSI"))
 (via (at 176.7 98.2) (size 0.6) (drill 0.3) (layers "F.Cu" "B.Cu") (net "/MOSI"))
 (segment (start 176.7 98.2) (end 166.925 98.2) (width 0.2) (layer "B.Cu") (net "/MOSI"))
 (segment (start 139.275 113.8) (end 168.075 113.8) (width 0.2) (layer "F.Cu") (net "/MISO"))
 (segment (start 175.9 105.975) (end 175.9 101.65) (width 0.2) (layer "F.Cu") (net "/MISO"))
 (segment (start 175.9 101.65) (end 174.99 100.74) (width 0.2) (layer "F.Cu") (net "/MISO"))
 (segment (start 168.075 113.8) (end 175.9 105.975) (width 0.2) (layer "F.Cu") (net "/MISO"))
 (segment (start 174.99 100.74) (end 166.925 100.74) (width 0.2) (layer "F.Cu") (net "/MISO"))
 (segment (start 136.5 111.025) (end 139.275 113.8) (width 0.2) (layer "F.Cu") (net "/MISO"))
 (segment (start 136.5 109.2) (end 136.5 111.025) (width 0.2) (layer "F.Cu") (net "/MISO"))
 (segment (start 144.9 111.5) (end 158.9 111.5) (width 0.2) (layer "F.Cu") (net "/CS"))
 (segment (start 136.5 93.96) (end 138.735 93.96) (width 0.2) (layer "F.Cu") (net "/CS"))
 (segment (start 163.65 106.75) (end 163.65 104.25) (width 0.2) (layer "F.Cu") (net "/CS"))
 (segment (start 163.65 104.25) (end 164.62 103.28) (width 0.2) (layer "F.Cu") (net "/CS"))
 (segment (start 141.125 107.725) (end 144.9 111.5) (width 0.2) (layer "F.Cu") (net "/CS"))
 (segment (start 164.62 103.28) (end 166.925 103.28) (width 0.2) (layer "F.Cu") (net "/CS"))
 (segment (start 158.9 111.5) (end 163.65 106.75) (width 0.2) (layer "F.Cu") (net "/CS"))
 (segment (start 138.735 93.96) (end 141.125 96.35) (width 0.2) (layer "F.Cu") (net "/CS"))
 (segment (start 141.125 96.35) (end 141.125 107.725) (width 0.2) (layer "F.Cu") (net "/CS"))
 (segment (start 170.05 110.9) (end 167.9 113.05) (width 0.2) (layer "F.Cu") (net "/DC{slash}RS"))
 (segment (start 170.05 109.5) (end 170.05 110.9) (width 0.2) (layer "F.Cu") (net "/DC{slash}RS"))
 (segment (start 139.65 99.85) (end 138.84 99.04) (width 0.2) (layer "F.Cu") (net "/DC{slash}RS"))
 (segment (start 139.65 108.35) (end 139.65 99.85) (width 0.2) (layer "F.Cu") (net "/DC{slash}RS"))
 (segment (start 144.35 113.05) (end 139.65 108.35) (width 0.2) (layer "F.Cu") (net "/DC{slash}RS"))
 (segment (start 168.91 108.36) (end 170.05 109.5) (width 0.2) (layer "F.Cu") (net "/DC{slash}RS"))
 (segment (start 167.9 113.05) (end 144.35 113.05) (width 0.2) (layer "F.Cu") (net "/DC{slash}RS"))
 (segment (start 138.84 99.04) (end 136.5 99.04) (width 0.2) (layer "F.Cu") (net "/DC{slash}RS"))
 (segment (start 166.925 108.36) (end 168.91 108.36) (width 0.2) (layer "F.Cu") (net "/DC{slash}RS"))
 (segment (start 144.55 112.15) (end 160.05 112.15) (width 0.2) (layer "F.Cu") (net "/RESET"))
 (segment (start 140.425 108.025) (end 144.55 112.15) (width 0.2) (layer "F.Cu") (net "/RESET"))
 (segment (start 161.3 110.9) (end 166.925 110.9) (width 0.2) (layer "F.Cu") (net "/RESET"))
 (segment (start 139.525 96.5) (end 140.425 97.4) (width 0.2) (layer "F.Cu") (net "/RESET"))
 (segment (start 160.05 112.15) (end 161.3 110.9) (width 0.2) (layer "F.Cu") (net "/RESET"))
 (segment (start 136.5 96.5) (end 139.525 96.5) (width 0.2) (layer "F.Cu") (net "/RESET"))
 (segment (start 140.425 97.4) (end 140.425 108.025) (width 0.2) (layer "F.Cu") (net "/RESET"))
 (segment (start 131.075 81.075) (end 131.075 112.525) (width 0.2) (layer "F.Cu") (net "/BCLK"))
 (segment (start 170.65 118.625) (end 178.375 110.9) (width 0.2) (layer "F.Cu") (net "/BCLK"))
 (segment (start 131.075 112.525) (end 137.175 118.625) (width 0.2) (layer "F.Cu") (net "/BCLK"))
 (segment (start 146.45 79) (end 133.15 79) (width 0.2) (layer "F.Cu") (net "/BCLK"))
 (segment (start 178.375 110.9) (end 184.705 110.9) (width 0.2) (layer "F.Cu") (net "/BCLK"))
 (segment (start 133.15 79) (end 131.075 81.075) (width 0.2) (layer "F.Cu") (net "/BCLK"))
 (segment (start 149.25 76.2) (end 146.45 79) (width 0.2) (layer "F.Cu") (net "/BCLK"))
 (segment (start 152.907 76.2) (end 149.25 76.2) (width 0.2) (layer "F.Cu") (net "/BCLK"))
 (segment (start 137.175 118.625) (end 170.65 118.625) (width 0.2) (layer "F.Cu") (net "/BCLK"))
 (segment (start 169.975 118.075) (end 179.69 108.36) (width 0.2) (layer "F.Cu") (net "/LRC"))
 (segment (start 137.45 118.075) (end 169.975 118.075) (width 0.2) (layer "F.Cu") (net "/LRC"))
 (segment (start 147.525 78.825) (end 146.6 79.75) (width 0.2) (layer "F.Cu") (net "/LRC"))
 (segment (start 131.725 112.35) (end 137.45 118.075) (width 0.2) (layer "F.Cu") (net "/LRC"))
 (segment (start 146.6 79.75) (end 133.5 79.75) (width 0.2) (layer "F.Cu") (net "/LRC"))
 (segment (start 152.907 78.74) (end 152.822 78.825) (width 0.2) (layer "F.Cu") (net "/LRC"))
 (segment (start 152.722 78.925) (end 152.907 78.74) (width 0.2) (layer "F.Cu") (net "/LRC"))
 (segment (start 179.69 108.36) (end 184.705 108.36) (width 0.2) (layer "F.Cu") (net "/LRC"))
 (segment (start 152.822 78.825) (end 147.525 78.825) (width 0.2) (layer "F.Cu") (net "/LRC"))
 (segment (start 133.5 79.75) (end 131.725 81.525) (width 0.2) (layer "F.Cu") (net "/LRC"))
 (segment (start 131.725 81.525) (end 131.725 112.35) (width 0.2) (layer "F.Cu") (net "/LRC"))
 (segment (start 153.8 80.525) (end 133.975 80.525) (width 0.2) (layer "F.Cu") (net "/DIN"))
 (segment (start 152.907 73.66) (end 155.81 73.66) (width 0.2) (layer "F.Cu") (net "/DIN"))
 (segment (start 133.975 80.525) (end 132.6 81.9) (width 0.2) (layer "F.Cu") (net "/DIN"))
 (segment (start 156.65 74.5) (end 156.65 77.675) (width 0.2) (layer "F.Cu") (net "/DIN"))
 (segment (start 132.6 112.225) (end 137.65 117.275) (width 0.2) (layer "F.Cu") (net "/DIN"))
 (segment (start 156.65 77.675) (end 153.8 80.525) (width 0.2) (layer "F.Cu") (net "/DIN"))
 (segment (start 137.65 117.275) (end 169.6 117.275) (width 0.2) (layer "F.Cu") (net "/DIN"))
 (segment (start 132.6 81.9) (end 132.6 112.225) (width 0.2) (layer "F.Cu") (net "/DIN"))
 (segment (start 155.81 73.66) (end 156.65 74.5) (width 0.2) (layer "F.Cu") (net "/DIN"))
 (segment (start 169.6 117.275) (end 183.595 103.28) (width 0.2) (layer "F.Cu") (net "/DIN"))
 (segment (start 183.595 103.28) (end 184.705 103.28) (width 0.2) (layer "F.Cu") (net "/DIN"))
 (segment (start 134.25 81.325) (end 154.275 81.325) (width 0.2) (layer "F.Cu") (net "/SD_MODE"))
 (segment (start 184.705 101.02) (end 169.225 116.5) (width 0.2) (layer "F.Cu") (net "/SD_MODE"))
 (segment (start 154.275 81.325) (end 157.475 78.125) (width 0.2) (layer "F.Cu") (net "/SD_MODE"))
 (segment (start 157.475 71.55) (end 154.525 68.6) (width 0.2) (layer "F.Cu") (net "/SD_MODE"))
 (segment (start 154.525 68.6) (end 152.927 68.6) (width 0.2) (layer "F.Cu") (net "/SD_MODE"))
 (segment (start 169.225 116.5) (end 137.95 116.5) (width 0.2) (layer "F.Cu") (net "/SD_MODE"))
 (segment (start 133.275 111.825) (end 133.275 82.3) (width 0.2) (layer "F.Cu") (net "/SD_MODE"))
 (segment (start 157.475 78.125) (end 157.475 71.55) (width 0.2) (layer "F.Cu") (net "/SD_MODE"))
 (segment (start 184.705 100.74) (end 184.705 101.02) (width 0.2) (layer "F.Cu") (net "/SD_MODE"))
 (segment (start 133.275 82.3) (end 134.25 81.325) (width 0.2) (layer "F.Cu") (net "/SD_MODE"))
 (segment (start 152.927 68.6) (end 152.907 68.58) (width 0.2) (layer "F.Cu") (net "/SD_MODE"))
 (segment (start 137.95 116.5) (end 133.275 111.825) (width 0.2) (layer "F.Cu") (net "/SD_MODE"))
 (segment (start 131.075 112.75) (end 131.075 90.725) (width 0.5) (layer "B.Cu") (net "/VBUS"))
 (segment (start 131.05 69.95) (end 137.5 63.5) (width 0.5) (layer "B.Cu") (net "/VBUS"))
 (segment (start 131.05 90.7) (end 131.05 69.95) (width 0.5) (layer "B.Cu") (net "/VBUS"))
 (segment (start 188.9 64.625) (end 188.9 117.025) (width 0.5) (layer "B.Cu") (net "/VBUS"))
 (segment (start 131.075 90.725) (end 131.05 90.7) (width 0.5) (layer "B.Cu") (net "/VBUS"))
 (segment (start 188.9 117.025) (end 187.55 118.375) (width 0.5) (layer "B.Cu") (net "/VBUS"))
 (segment (start 131.075 90.725) (end 132.92 88.88) (width 0.5) (layer "B.Cu") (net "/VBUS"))
 (segment (start 132.92 88.88) (end 136.5 88.88) (width 0.5) (layer "B.Cu") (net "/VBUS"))
 (segment (start 136.7 118.375) (end 131.075 112.75) (width 0.5) (layer "B.Cu") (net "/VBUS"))
 (segment (start 137.5 63.5) (end 152.907 63.5) (width 0.5) (layer "B.Cu") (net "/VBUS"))
 (segment (start 187.55 118.375) (end 136.7 118.375) (width 0.5) (layer "B.Cu") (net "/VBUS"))
 (segment (start 186.915 62.64) (end 188.9 64.625) (width 0.5) (layer "B.Cu") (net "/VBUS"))
 (segment (start 184.705 62.64) (end 186.915 62.64) (width 0.5) (layer "B.Cu") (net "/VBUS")))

